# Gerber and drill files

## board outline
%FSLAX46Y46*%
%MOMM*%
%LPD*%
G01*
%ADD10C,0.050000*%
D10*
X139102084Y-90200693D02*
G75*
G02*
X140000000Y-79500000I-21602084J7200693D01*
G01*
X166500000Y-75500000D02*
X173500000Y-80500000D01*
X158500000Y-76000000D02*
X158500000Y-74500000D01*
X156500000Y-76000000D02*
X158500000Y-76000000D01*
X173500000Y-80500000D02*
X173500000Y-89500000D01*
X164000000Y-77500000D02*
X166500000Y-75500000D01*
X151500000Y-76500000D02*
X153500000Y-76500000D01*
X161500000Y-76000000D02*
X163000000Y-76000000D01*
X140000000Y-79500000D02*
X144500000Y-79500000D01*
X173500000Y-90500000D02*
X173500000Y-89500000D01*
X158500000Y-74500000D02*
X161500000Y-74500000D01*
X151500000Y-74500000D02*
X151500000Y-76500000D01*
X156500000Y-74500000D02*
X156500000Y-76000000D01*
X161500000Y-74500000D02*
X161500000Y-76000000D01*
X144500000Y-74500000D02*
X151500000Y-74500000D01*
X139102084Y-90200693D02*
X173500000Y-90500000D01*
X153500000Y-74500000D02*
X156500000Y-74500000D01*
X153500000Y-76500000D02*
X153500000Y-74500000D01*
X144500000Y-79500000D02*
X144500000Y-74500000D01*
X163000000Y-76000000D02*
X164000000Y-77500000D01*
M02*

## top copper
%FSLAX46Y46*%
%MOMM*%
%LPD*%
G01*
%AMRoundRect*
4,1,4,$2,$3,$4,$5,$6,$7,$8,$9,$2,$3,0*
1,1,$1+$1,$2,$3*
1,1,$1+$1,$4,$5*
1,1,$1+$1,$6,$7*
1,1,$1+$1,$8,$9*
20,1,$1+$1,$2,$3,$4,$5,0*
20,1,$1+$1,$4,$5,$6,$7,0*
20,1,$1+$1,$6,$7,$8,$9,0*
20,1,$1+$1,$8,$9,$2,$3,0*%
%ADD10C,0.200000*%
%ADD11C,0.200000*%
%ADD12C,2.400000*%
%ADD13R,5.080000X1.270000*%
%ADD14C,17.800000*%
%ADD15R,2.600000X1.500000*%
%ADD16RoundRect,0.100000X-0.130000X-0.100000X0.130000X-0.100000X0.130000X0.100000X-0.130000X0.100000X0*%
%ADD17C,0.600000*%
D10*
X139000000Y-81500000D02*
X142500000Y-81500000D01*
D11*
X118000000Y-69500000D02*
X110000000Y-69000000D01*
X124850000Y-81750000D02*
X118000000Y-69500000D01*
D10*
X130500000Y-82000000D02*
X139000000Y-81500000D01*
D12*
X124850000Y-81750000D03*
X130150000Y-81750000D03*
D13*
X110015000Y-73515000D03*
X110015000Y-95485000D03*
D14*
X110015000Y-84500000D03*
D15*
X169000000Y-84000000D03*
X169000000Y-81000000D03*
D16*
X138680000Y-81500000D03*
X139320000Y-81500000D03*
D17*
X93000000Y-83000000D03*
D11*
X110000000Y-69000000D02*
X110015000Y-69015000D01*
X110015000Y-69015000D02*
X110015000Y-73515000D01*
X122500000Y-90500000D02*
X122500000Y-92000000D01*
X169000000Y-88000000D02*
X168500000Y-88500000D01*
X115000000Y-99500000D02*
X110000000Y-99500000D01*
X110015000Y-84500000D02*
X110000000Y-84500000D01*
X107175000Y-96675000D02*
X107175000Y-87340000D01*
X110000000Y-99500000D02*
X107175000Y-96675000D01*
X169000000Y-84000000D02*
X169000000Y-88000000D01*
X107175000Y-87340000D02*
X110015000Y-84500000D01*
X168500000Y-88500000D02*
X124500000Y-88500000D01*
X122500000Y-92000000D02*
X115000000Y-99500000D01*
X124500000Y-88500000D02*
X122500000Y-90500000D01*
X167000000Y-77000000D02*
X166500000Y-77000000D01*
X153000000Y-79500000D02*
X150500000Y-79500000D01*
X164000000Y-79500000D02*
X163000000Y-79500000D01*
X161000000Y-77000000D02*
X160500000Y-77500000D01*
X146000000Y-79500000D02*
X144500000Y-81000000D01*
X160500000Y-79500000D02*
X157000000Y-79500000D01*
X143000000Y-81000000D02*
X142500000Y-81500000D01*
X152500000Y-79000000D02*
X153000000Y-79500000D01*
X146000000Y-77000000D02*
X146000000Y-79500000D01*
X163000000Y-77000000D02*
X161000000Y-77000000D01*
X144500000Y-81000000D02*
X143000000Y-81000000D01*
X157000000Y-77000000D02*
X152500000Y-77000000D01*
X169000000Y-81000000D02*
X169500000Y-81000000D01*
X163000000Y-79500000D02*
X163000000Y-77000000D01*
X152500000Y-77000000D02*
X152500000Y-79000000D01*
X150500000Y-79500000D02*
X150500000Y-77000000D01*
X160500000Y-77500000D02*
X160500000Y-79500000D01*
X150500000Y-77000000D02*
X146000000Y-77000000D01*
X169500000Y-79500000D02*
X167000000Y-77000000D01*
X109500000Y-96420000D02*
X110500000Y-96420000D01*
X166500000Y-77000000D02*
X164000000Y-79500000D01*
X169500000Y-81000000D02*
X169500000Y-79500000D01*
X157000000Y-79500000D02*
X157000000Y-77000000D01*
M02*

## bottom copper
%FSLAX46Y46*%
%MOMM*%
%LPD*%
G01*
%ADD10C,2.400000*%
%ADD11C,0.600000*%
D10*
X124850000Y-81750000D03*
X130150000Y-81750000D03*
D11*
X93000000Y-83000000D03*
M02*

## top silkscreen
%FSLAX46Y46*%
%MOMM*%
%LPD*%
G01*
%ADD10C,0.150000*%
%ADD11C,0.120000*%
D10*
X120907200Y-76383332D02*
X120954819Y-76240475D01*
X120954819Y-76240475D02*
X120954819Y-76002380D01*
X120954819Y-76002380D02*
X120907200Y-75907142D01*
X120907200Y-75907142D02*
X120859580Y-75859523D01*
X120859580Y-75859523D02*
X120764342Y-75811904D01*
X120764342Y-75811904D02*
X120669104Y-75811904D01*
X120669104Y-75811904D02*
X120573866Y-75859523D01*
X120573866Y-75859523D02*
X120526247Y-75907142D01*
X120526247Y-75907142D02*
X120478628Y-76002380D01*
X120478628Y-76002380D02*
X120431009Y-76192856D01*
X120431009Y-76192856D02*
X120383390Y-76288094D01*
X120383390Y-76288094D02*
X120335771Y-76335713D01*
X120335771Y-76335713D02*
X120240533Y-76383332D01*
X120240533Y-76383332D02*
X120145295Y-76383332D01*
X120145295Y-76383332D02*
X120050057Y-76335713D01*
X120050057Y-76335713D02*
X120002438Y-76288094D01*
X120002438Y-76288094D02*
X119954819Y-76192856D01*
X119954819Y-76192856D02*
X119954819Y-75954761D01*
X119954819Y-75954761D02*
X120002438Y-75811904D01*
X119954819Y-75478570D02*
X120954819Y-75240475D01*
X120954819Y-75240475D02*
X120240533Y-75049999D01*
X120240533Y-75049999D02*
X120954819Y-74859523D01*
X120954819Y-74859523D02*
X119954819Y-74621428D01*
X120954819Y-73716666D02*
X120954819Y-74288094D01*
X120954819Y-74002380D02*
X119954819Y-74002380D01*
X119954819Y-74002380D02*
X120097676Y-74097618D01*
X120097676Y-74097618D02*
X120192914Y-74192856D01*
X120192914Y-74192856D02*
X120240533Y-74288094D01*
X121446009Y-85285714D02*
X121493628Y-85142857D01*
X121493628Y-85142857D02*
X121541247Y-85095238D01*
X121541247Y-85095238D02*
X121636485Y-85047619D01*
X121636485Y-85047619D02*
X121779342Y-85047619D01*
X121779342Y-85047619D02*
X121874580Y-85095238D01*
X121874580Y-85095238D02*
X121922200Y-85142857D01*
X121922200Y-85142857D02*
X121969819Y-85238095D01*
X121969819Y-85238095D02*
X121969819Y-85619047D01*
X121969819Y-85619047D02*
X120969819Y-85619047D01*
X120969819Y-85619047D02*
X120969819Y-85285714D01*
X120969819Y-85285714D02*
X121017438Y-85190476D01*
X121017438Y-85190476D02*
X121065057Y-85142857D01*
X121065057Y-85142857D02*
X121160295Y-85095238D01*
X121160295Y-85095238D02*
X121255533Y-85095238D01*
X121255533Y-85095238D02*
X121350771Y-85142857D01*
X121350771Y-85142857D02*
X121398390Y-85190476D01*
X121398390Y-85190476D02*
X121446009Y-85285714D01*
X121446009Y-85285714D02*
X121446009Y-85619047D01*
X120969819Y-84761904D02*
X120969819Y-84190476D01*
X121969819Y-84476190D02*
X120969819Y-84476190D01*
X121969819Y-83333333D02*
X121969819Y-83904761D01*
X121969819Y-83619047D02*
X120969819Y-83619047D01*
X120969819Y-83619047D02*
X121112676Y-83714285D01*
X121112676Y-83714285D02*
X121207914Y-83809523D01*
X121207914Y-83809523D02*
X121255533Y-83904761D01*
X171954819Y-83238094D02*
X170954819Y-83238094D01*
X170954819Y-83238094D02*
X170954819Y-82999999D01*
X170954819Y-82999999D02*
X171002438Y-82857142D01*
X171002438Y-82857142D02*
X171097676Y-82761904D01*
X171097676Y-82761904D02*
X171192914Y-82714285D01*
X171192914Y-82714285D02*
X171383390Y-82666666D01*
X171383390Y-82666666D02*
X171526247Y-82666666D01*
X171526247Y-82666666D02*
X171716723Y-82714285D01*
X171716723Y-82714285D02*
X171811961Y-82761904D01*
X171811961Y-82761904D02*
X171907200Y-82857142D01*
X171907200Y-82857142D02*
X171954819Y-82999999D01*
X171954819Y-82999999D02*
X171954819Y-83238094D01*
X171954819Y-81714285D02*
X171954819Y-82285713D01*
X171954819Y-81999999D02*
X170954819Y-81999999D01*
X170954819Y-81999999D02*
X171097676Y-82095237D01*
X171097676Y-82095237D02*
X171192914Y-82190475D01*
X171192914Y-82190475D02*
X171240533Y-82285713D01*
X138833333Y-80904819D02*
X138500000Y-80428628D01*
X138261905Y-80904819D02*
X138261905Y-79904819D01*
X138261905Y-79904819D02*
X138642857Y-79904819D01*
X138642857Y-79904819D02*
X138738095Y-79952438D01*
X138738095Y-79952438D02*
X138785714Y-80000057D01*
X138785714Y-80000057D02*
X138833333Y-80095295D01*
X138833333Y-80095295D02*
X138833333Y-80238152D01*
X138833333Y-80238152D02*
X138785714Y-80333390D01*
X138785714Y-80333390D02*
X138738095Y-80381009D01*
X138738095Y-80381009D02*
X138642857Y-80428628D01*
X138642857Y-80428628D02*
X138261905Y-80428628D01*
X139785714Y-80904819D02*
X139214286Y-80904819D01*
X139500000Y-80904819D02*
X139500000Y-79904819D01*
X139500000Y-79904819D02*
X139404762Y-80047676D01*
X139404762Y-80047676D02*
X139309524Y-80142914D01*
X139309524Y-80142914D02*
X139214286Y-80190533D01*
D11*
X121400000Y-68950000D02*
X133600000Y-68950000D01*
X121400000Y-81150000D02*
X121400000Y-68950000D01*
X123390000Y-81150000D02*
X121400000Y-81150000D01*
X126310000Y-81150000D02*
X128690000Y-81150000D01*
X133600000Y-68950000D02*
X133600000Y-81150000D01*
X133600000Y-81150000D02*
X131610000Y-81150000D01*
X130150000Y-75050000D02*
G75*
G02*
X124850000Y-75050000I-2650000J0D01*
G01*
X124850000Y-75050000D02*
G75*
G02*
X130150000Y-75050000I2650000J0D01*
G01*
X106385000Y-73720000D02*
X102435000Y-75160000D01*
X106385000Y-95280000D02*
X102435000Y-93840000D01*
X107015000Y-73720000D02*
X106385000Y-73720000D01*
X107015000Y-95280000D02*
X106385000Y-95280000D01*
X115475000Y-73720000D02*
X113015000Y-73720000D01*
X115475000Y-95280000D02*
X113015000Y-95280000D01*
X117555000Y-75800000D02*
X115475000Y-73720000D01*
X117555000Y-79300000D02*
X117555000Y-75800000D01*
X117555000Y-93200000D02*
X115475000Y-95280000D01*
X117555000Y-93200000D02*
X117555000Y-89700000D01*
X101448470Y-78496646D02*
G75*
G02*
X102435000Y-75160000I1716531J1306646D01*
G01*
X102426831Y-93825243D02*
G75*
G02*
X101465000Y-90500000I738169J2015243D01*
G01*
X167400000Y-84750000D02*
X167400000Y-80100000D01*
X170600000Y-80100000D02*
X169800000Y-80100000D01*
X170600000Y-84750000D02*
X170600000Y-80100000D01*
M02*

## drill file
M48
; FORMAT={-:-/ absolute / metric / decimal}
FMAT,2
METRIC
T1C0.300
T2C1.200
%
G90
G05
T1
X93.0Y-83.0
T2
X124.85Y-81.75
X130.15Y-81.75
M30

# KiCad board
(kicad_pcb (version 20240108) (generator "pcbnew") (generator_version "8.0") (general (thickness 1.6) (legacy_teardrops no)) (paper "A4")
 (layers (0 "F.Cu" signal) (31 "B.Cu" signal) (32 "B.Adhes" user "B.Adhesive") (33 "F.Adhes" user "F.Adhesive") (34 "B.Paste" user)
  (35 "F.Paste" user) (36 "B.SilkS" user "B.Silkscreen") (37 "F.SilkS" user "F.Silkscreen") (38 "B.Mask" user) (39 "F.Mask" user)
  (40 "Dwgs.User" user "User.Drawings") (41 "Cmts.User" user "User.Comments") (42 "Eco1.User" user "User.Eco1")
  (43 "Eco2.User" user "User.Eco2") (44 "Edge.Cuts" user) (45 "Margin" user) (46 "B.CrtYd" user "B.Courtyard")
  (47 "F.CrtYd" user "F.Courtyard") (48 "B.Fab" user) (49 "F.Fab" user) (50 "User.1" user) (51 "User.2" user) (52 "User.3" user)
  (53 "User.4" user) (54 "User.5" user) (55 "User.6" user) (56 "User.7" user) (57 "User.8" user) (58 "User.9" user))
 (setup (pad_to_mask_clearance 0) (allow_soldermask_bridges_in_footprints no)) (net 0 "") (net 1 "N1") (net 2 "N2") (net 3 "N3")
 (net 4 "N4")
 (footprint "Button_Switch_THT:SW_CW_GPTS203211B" (layer "F.Cu") (at 124.85 81.75 90)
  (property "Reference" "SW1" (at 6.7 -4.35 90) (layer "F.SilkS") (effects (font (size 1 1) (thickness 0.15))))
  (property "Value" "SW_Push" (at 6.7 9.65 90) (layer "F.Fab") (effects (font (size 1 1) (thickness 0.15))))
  (fp_line (start 12.8 -3.45) (end 12.8 8.75) (stroke (width 0.12) (type solid)) (layer "F.SilkS"))
  (fp_line (start 0.6 -3.45) (end 12.8 -3.45) (stroke (width 0.12) (type solid)) (layer "F.SilkS"))
  (fp_line (start 0.6 -1.46) (end 0.6 -3.45) (stroke (width 0.12) (type solid)) (layer "F.SilkS"))
  (fp_line (start 0.6 1.46) (end 0.6 3.84) (stroke (width 0.12) (type solid)) (layer "F.SilkS"))
  (fp_line (start 12.8 8.75) (end 0.6 8.75) (stroke (width 0.12) (type solid)) (layer "F.SilkS"))
  (fp_line (start 0.6 8.75) (end 0.6 6.76) (stroke (width 0.12) (type solid)) (layer "F.SilkS"))
  (fp_circle (center 6.7 2.65) (end 9.35 2.65) (stroke (width 0.12) (type solid)) (fill none) (layer "F.SilkS"))
  (pad "1" thru_hole circle (at 0 0 90) (size 2.4 2.4) (drill 1.2) (layers "*.Cu" "*.Mask") (remove_unused_layers no) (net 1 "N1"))
  (pad "2" thru_hole circle (at 0 5.3 90) (size 2.4 2.4) (drill 1.2) (layers "*.Cu" "*.Mask") (remove_unused_layers no) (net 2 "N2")))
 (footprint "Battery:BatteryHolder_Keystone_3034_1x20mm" (layer "F.Cu") (at 110.015 84.5 -90)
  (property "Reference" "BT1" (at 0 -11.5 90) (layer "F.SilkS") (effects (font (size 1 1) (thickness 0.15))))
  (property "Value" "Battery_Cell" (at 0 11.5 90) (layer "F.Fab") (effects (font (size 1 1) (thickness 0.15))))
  (fp_line (start -10.78 3.63) (end -9.34 7.58) (stroke (width 0.12) (type solid)) (layer "F.SilkS"))
  (fp_line (start 10.78 3.63) (end 9.34 7.58) (stroke (width 0.12) (type solid)) (layer "F.SilkS"))
  (fp_line (start -10.78 3) (end -10.78 3.63) (stroke (width 0.12) (type solid)) (layer "F.SilkS"))
  (fp_line (start 10.78 3) (end 10.78 3.63) (stroke (width 0.12) (type solid)) (layer "F.SilkS"))
  (fp_line (start -10.78 -5.46) (end -10.78 -3) (stroke (width 0.12) (type solid)) (layer "F.SilkS"))
  (fp_line (start 10.78 -5.46) (end 10.78 -3) (stroke (width 0.12) (type solid)) (layer "F.SilkS"))
  (fp_line (start -8.7 -7.54) (end -10.78 -5.46) (stroke (width 0.12) (type solid)) (layer "F.SilkS"))
  (fp_line (start -5.2 -7.54) (end -8.7 -7.54) (stroke (width 0.12) (type solid)) (layer "F.SilkS"))
  (fp_line (start 8.7 -7.54) (end 10.78 -5.46) (stroke (width 0.12) (type solid)) (layer "F.SilkS"))
  (fp_line (start 8.7 -7.54) (end 5.2 -7.54) (stroke (width 0.12) (type solid)) (layer "F.SilkS"))
  (fp_arc (start -6.003354 8.56653) (mid -7.921654 8.918738) (end -9.34 7.58) (stroke (width 0.12) (type solid)) (layer "F.SilkS"))
  (fp_arc (start 9.325243 7.588169) (mid 7.90634 8.911668) (end 6 8.55) (stroke (width 0.12) (type solid)) (layer "F.SilkS"))
  (pad "1" smd rect (at -10.985 0 270) (size 1.27 5.08) (layers "F.Cu" "F.Paste" "F.Mask") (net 1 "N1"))
  (pad "1" smd rect (at 10.985 0 270) (size 1.27 5.08) (layers "F.Cu" "F.Paste" "F.Mask") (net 1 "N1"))
  (pad "2" smd circle (at 0 0 270) (size 17.8 17.8) (layers "F.Cu" "F.Mask") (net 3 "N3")))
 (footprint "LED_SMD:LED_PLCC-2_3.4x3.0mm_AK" (layer "F.Cu") (at 169 82.5 -90)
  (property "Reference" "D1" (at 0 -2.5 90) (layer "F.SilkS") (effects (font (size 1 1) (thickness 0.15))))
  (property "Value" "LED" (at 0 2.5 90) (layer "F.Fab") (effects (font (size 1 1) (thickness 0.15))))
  (fp_line (start 2.25 1.6) (end -2.4 1.6) (stroke (width 0.12) (type solid)) (layer "F.SilkS"))
  (fp_line (start -2.4 -1.6) (end -2.4 -0.8) (stroke (width 0.12) (type solid)) (layer "F.SilkS"))
  (fp_line (start 2.25 -1.6) (end -2.4 -1.6) (stroke (width 0.12) (type solid)) (layer "F.SilkS"))
  (pad "1" smd rect (at 1.5 0 270) (size 1.5 2.6) (layers "F.Cu" "F.Paste" "F.Mask") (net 3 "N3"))
  (pad "2" smd rect (at -1.5 0 270) (size 1.5 2.6) (layers "F.Cu" "F.Paste" "F.Mask") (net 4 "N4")))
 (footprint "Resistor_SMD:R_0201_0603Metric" (layer "F.Cu") (at 139 81.5)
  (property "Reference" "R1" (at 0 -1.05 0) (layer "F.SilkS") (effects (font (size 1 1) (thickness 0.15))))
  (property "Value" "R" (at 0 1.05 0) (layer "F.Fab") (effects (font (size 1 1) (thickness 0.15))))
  (pad "" smd roundrect (at -0.345 0) (size 0.318 0.36) (layers "F.Paste") (roundrect_rratio 0.25))
  (pad "" smd roundrect (at 0.345 0) (size 0.318 0.36) (layers "F.Paste") (roundrect_rratio 0.25))
  (pad "1" smd roundrect (at -0.32 0) (size 0.46 0.4) (layers "F.Cu" "F.Mask") (roundrect_rratio 0.25) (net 2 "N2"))
  (pad "2" smd roundrect (at 0.32 0) (size 0.46 0.4) (layers "F.Cu" "F.Mask") (roundrect_rratio 0.25) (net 4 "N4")))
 (gr_line (start 139 81.5) (end 142.5 81.5) (stroke (width 0.2) (type default)) (layer "F.Cu"))
 (gr_line (start 118 69.5) (end 110 69) (stroke (width 0.2) (type default)) (layer "F.Cu") (net 1))
 (gr_line (start 124.85 81.75) (end 118 69.5) (stroke (width 0.2) (type default)) (layer "F.Cu") (net 1))
 (gr_line (start 130.5 82) (end 139 81.5) (stroke (width 0.2) (type default)) (layer "F.Cu"))
 (gr_arc (start 139.102084 90.200693) (mid 94.80915 81.095966) (end 140 79.5) (stroke (width 0.05) (type default)) (layer "Edge.Cuts"))
 (gr_line (start 166.5 75.5) (end 173.5 80.5) (stroke (width 0.05) (type default)) (layer "Edge.Cuts"))
 (gr_line (start 158.5 76) (end 158.5 74.5) (stroke (width 0.05) (type default)) (layer "Edge.Cuts"))
 (gr_line (start 156.5 76) (end 158.5 76) (stroke (width 0.05) (type default)) (layer "Edge.Cuts"))
 (gr_line (start 173.5 80.5) (end 173.5 89.5) (stroke (width 0.05) (type default)) (layer "Edge.Cuts"))
 (gr_line (start 164 77.5) (end 166.5 75.5) (stroke (width 0.05) (type default)) (layer "Edge.Cuts"))
 (gr_line (start 151.5 76.5) (end 153.5 76.5) (stroke (width 0.05) (type default)) (layer "Edge.Cuts"))
 (gr_line (start 161.5 76) (end 163 76) (stroke (width 0.05) (type default)) (layer "Edge.Cuts"))
 (gr_line (start 140 79.5) (end 144.5 79.5) (stroke (width 0.05) (type default)) (layer "Edge.Cuts"))
 (gr_line (start 173.5 90.5) (end 173.5 89.5) (stroke (width 0.05) (type default)) (layer "Edge.Cuts"))
 (gr_line (start 158.5 74.5) (end 161.5 74.5) (stroke (width 0.05) (type default)) (layer "Edge.Cuts"))
 (gr_line (start 151.5 74.5) (end 151.5 76.5) (stroke (width 0.05) (type default)) (layer "Edge.Cuts"))
 (gr_line (start 156.5 74.5) (end 156.5 76) (stroke (width 0.05) (type default)) (layer "Edge.Cuts"))
 (gr_line (start 161.5 74.5) (end 161.5 76) (stroke (width 0.05) (type default)) (layer "Edge.Cuts"))
 (gr_line (start 144.5 74.5) (end 151.5 74.5) (stroke (width 0.05) (type default)) (layer "Edge.Cuts"))
 (gr_line (start 139.102084 90.200693) (end 173.5 90.5) (stroke (width 0.05) (type default)) (layer "Edge.Cuts"))
 (gr_line (start 153.5 74.5) (end 156.5 74.5) (stroke (width 0.05) (type default)) (layer "Edge.Cuts"))
 (gr_line (start 153.5 76.5) (end 153.5 74.5) (stroke (width 0.05) (type default)) (layer "Edge.Cuts"))
 (gr_line (start 144.5 79.5) (end 144.5 74.5) (stroke (width 0.05) (type default)) (layer "Edge.Cuts"))
 (gr_line (start 163 76) (end 164 77.5) (stroke (width 0.05) (type default)) (layer "Edge.Cuts"))
 (via (at 93 83) (size 0.6) (drill 0.3) (layers "F.Cu" "B.Cu") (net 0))
 (segment (start 110 69) (end 110.015 69.015) (width 0.2) (layer "F.Cu") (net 1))
 (segment (start 110.015 69.015) (end 110.015 73.515) (width 0.2) (layer "F.Cu") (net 1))
 (segment (start 122.5 90.5) (end 122.5 92) (width 0.2) (layer "F.Cu") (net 3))
 (segment (start 169 88) (end 168.5 88.5) (width 0.2) (layer "F.Cu") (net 3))
 (segment (start 115 99.5) (end 110 99.5) (width 0.2) (layer "F.Cu") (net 3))
 (segment (start 110.015 84.5) (end 110 84.5) (width 0.2) (layer "F.Cu") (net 3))
 (segment (start 107.175 96.675) (end 107.175 87.34) (width 0.2) (layer "F.Cu") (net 3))
 (segment (start 110 99.5) (end 107.175 96.675) (width 0.2) (layer "F.Cu") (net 3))
 (segment (start 169 84) (end 169 88) (width 0.2) (layer "F.Cu") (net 3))
 (segment (start 107.175 87.34) (end 110.015 84.5) (width 0.2) (layer "F.Cu") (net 3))
 (segment (start 168.5 88.5) (end 124.5 88.5) (width 0.2) (layer "F.Cu") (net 3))
 (segment (start 122.5 92) (end 115 99.5) (width 0.2) (layer "F.Cu") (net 3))
 (segment (start 124.5 88.5) (end 122.5 90.5) (width 0.2) (layer "F.Cu") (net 3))
 (segment (start 167 77) (end 166.5 77) (width 0.2) (layer "F.Cu") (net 4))
 (segment (start 153 79.5) (end 150.5 79.5) (width 0.2) (layer "F.Cu") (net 4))
 (segment (start 164 79.5) (end 163 79.5) (width 0.2) (layer "F.Cu") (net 4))
 (segment (start 161 77) (end 160.5 77.5) (width 0.2) (layer "F.Cu") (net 4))
 (segment (start 146 79.5) (end 144.5 81) (width 0.2) (layer "F.Cu") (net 4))
 (segment (start 160.5 79.5) (end 157 79.5) (width 0.2) (layer "F.Cu") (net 4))
 (segment (start 143 81) (end 142.5 81.5) (width 0.2) (layer "F.Cu") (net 4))
 (segment (start 152.5 79) (end 153 79.5) (width 0.2) (layer "F.Cu") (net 4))
 (segment (start 146 77) (end 146 79.5) (width 0.2) (layer "F.Cu") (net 4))
 (segment (start 163 77) (end 161 77) (width 0.2) (layer "F.Cu") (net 4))
 (segment (start 144.5 81) (end 143 81) (width 0.2) (layer "F.Cu") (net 4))
 (segment (start 157 77) (end 152.5 77) (width 0.2) (layer "F.Cu") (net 4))
 (segment (start 169 81) (end 169.5 81) (width 0.2) (layer "F.Cu") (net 4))
 (segment (start 163 79.5) (end 163 77) (width 0.2) (layer "F.Cu") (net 4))
 (segment (start 152.5 77) (end 152.5 79) (width 0.2) (layer "F.Cu") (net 4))
 (segment (start 150.5 79.5) (end 150.5 77) (width 0.2) (layer "F.Cu") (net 4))
 (segment (start 160.5 77.5) (end 160.5 79.5) (width 0.2) (layer "F.Cu") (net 4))
 (segment (start 150.5 77) (end 146 77) (width 0.2) (layer "F.Cu") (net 4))
 (segment (start 169.5 79.5) (end 167 77) (width 0.2) (layer "F.Cu") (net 4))
 (segment (start 109.5 96.42) (end 110.5 96.42) (width 0.2) (layer "F.Cu") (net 4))
 (segment (start 166.5 77) (end 164 79.5) (width 0.2) (layer "F.Cu") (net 4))
 (segment (start 169.5 81) (end 169.5 79.5) (width 0.2) (layer "F.Cu") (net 4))
 (segment (start 157 79.5) (end 157 77) (width 0.2) (layer "F.Cu") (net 4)))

